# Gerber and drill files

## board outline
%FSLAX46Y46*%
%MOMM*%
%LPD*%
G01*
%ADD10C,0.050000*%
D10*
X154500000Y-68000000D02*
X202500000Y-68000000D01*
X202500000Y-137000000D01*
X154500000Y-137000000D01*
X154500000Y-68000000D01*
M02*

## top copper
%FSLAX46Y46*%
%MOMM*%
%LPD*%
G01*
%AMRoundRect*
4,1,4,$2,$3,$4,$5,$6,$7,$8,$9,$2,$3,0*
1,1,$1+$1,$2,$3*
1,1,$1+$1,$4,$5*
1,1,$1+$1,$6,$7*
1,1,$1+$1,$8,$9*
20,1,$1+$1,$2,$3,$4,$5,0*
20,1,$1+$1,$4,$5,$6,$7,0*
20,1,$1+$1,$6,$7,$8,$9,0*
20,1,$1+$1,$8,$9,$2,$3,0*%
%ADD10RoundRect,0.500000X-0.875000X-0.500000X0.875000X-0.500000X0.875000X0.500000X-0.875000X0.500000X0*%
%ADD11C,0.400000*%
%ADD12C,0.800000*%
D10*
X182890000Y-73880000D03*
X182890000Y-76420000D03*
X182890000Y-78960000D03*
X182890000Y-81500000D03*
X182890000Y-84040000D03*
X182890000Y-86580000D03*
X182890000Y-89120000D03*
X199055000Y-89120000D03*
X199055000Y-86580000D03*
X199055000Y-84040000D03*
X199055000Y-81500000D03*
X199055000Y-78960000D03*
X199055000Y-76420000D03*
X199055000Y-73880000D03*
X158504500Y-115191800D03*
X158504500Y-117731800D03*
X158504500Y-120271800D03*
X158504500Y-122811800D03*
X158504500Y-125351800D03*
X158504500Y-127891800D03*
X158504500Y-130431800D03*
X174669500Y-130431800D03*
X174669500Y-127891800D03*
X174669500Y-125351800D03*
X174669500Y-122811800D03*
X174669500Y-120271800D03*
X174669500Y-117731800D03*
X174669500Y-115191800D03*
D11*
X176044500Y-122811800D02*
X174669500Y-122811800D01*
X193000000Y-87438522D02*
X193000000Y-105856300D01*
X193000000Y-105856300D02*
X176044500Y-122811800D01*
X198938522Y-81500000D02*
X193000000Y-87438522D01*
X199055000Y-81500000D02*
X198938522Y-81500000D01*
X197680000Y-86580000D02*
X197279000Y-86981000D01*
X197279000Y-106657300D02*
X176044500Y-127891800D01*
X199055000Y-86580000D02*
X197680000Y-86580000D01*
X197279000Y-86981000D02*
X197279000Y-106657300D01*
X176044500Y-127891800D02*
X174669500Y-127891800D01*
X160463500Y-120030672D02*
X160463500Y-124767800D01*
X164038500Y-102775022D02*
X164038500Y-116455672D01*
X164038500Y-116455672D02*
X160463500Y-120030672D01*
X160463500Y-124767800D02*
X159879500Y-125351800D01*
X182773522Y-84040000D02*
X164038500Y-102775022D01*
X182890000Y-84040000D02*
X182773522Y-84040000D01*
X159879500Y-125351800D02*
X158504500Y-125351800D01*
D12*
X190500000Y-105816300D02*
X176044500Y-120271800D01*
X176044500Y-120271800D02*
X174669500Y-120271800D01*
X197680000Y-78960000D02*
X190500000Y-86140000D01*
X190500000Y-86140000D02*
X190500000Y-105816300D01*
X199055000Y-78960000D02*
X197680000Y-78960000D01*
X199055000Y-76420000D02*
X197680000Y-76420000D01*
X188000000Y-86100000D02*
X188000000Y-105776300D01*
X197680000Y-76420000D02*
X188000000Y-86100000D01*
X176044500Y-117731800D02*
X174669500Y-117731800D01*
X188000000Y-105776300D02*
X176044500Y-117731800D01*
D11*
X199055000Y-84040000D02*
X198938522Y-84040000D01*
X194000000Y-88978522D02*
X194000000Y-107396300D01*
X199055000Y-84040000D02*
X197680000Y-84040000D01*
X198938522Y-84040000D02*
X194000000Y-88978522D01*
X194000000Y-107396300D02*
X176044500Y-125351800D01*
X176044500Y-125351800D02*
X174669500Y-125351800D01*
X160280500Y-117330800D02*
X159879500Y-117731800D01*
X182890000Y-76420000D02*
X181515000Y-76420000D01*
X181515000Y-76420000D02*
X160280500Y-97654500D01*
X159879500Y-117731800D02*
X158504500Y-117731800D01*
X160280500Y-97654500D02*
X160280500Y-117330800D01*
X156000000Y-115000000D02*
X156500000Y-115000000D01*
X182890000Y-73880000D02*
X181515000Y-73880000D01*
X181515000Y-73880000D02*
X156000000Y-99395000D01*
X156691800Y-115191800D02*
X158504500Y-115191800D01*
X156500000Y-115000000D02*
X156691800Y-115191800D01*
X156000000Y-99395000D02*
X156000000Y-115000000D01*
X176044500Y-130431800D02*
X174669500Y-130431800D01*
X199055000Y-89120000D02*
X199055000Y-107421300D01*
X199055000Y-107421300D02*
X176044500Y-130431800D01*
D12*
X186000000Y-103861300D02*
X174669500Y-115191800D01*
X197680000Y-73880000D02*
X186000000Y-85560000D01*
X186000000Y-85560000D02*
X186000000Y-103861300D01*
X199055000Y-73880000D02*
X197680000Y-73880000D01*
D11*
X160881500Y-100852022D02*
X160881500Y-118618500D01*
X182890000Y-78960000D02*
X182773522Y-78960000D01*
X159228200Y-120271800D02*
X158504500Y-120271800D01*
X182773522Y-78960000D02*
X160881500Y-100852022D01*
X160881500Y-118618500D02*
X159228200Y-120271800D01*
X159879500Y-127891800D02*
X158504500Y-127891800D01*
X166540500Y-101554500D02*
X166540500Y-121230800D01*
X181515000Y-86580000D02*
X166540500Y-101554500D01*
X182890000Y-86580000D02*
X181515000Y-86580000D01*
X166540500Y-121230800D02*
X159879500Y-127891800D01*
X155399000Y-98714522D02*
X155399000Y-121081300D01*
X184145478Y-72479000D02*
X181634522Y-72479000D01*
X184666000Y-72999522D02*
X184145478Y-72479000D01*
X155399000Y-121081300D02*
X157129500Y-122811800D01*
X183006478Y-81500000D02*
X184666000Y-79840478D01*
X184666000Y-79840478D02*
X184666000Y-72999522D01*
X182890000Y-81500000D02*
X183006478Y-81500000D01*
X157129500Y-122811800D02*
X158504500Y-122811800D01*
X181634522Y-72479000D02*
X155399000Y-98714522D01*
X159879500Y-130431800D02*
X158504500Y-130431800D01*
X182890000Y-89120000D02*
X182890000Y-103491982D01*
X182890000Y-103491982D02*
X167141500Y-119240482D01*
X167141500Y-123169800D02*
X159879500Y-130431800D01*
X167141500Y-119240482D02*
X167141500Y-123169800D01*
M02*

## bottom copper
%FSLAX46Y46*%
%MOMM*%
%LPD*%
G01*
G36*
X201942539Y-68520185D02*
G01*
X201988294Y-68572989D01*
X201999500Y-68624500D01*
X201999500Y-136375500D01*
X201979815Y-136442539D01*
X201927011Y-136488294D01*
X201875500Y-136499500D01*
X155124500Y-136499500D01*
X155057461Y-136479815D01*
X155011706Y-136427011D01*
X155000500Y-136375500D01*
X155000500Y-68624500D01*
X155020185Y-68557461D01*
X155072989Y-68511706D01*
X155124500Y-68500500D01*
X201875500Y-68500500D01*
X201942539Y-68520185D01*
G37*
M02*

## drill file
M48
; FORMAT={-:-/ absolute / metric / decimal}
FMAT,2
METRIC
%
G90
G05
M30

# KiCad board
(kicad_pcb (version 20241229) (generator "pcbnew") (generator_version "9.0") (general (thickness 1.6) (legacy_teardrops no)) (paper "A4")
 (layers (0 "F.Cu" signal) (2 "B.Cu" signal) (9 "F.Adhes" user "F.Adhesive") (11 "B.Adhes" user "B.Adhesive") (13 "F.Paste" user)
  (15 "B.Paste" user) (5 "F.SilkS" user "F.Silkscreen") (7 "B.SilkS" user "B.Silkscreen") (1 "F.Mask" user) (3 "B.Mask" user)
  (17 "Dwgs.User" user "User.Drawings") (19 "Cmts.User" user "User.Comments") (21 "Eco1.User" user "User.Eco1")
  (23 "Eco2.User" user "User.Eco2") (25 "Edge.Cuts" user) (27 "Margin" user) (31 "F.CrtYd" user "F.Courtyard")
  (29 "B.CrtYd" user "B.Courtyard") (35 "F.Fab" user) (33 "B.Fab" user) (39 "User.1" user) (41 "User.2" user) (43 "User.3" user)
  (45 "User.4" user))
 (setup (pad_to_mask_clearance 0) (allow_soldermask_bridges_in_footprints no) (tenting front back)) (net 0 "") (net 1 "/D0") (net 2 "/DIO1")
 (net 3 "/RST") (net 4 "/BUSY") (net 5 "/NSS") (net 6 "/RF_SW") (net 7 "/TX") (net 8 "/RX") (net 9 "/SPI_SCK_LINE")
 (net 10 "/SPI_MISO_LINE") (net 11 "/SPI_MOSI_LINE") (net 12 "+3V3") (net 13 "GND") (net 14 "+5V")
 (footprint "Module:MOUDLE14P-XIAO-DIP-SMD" (layer "F.Cu") (at 191 81.5)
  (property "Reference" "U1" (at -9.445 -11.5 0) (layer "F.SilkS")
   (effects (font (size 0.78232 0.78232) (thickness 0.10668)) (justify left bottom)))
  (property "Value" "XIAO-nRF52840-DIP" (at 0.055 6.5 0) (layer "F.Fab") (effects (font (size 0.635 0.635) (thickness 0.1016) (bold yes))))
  (pad "1" smd roundrect (at -8.11 -7.62) (size 2.75 2) (layers "F.Cu" "F.Mask" "F.Paste") (roundrect_rratio 0.25) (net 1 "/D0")
   (solder_mask_margin 0.0508) (thermal_bridge_angle 45))
  (pad "2" smd roundrect (at -8.11 -5.08) (size 2.75 2) (layers "F.Cu" "F.Mask" "F.Paste") (roundrect_rratio 0.25) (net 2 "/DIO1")
   (solder_mask_margin 0.0508) (thermal_bridge_angle 45))
  (pad "3" smd roundrect (at -8.11 -2.54) (size 2.75 2) (layers "F.Cu" "F.Mask" "F.Paste") (roundrect_rratio 0.25) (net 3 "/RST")
   (solder_mask_margin 0.0508) (thermal_bridge_angle 45))
  (pad "4" smd roundrect (at -8.11 0) (size 2.75 2) (layers "F.Cu" "F.Mask" "F.Paste") (roundrect_rratio 0.25) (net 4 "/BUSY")
   (solder_mask_margin 0.0508) (thermal_bridge_angle 45))
  (pad "5" smd roundrect (at -8.11 2.54) (size 2.75 2) (layers "F.Cu" "F.Mask" "F.Paste") (roundrect_rratio 0.25) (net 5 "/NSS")
   (solder_mask_margin 0.0508) (thermal_bridge_angle 45))
  (pad "6" smd roundrect (at -8.11 5.08) (size 2.75 2) (layers "F.Cu" "F.Mask" "F.Paste") (roundrect_rratio 0.25) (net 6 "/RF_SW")
   (solder_mask_margin 0.0508) (thermal_bridge_angle 45))
  (pad "7" smd roundrect (at -8.11 7.62) (size 2.75 2) (layers "F.Cu" "F.Mask" "F.Paste") (roundrect_rratio 0.25) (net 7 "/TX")
   (solder_mask_margin 0.0508) (thermal_bridge_angle 45))
  (pad "8" smd roundrect (at 8.055 7.62) (size 2.75 2) (layers "F.Cu" "F.Mask" "F.Paste") (roundrect_rratio 0.25) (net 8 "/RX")
   (solder_mask_margin 0.0508) (thermal_bridge_angle 45))
  (pad "9" smd roundrect (at 8.055 5.08) (size 2.75 2) (layers "F.Cu" "F.Mask" "F.Paste") (roundrect_rratio 0.25) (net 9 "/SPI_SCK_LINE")
   (solder_mask_margin 0.0508) (thermal_bridge_angle 45))
  (pad "10" smd roundrect (at 8.055 2.54) (size 2.75 2) (layers "F.Cu" "F.Mask" "F.Paste") (roundrect_rratio 0.25) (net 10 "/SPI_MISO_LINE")
   (solder_mask_margin 0.0508) (thermal_bridge_angle 45))
  (pad "11" smd roundrect (at 8.055 0) (size 2.75 2) (layers "F.Cu" "F.Mask" "F.Paste") (roundrect_rratio 0.25) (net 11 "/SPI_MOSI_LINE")
   (solder_mask_margin 0.0508) (thermal_bridge_angle 45))
  (pad "12" smd roundrect (at 8.055 -2.54) (size 2.75 2) (layers "F.Cu" "F.Mask" "F.Paste") (roundrect_rratio 0.25) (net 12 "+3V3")
   (solder_mask_margin 0.0508) (thermal_bridge_angle 45))
  (pad "13" smd roundrect (at 8.055 -5.08) (size 2.75 2) (layers "F.Cu" "F.Mask" "F.Paste") (roundrect_rratio 0.25) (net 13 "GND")
   (solder_mask_margin 0.0508) (thermal_bridge_angle 45))
  (pad "14" smd roundrect (at 8.055 -7.62) (size 2.75 2) (layers "F.Cu" "F.Mask" "F.Paste") (roundrect_rratio 0.25) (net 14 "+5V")
   (solder_mask_margin 0.0508) (thermal_bridge_angle 45)))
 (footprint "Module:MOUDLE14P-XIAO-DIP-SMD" (layer "F.Cu") (at 166.6145 122.8118)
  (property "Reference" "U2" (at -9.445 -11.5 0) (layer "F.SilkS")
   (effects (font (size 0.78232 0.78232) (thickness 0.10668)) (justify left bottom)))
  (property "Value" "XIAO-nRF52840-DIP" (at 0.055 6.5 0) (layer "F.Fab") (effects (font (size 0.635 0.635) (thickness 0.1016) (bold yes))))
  (pad "1" smd roundrect (at -8.11 -7.62) (size 2.75 2) (layers "F.Cu" "F.Mask" "F.Paste") (roundrect_rratio 0.25) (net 1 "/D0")
   (solder_mask_margin 0.0508) (thermal_bridge_angle 45))
  (pad "2" smd roundrect (at -8.11 -5.08) (size 2.75 2) (layers "F.Cu" "F.Mask" "F.Paste") (roundrect_rratio 0.25) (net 2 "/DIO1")
   (solder_mask_margin 0.0508) (thermal_bridge_angle 45))
  (pad "3" smd roundrect (at -8.11 -2.54) (size 2.75 2) (layers "F.Cu" "F.Mask" "F.Paste") (roundrect_rratio 0.25) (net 3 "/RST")
   (solder_mask_margin 0.0508) (thermal_bridge_angle 45))
  (pad "4" smd roundrect (at -8.11 0) (size 2.75 2) (layers "F.Cu" "F.Mask" "F.Paste") (roundrect_rratio 0.25) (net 4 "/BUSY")
   (solder_mask_margin 0.0508) (thermal_bridge_angle 45))
  (pad "5" smd roundrect (at -8.11 2.54) (size 2.75 2) (layers "F.Cu" "F.Mask" "F.Paste") (roundrect_rratio 0.25) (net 5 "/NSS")
   (solder_mask_margin 0.0508) (thermal_bridge_angle 45))
  (pad "6" smd roundrect (at -8.11 5.08) (size 2.75 2) (layers "F.Cu" "F.Mask" "F.Paste") (roundrect_rratio 0.25) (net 6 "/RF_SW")
   (solder_mask_margin 0.0508) (thermal_bridge_angle 45))
  (pad "7" smd roundrect (at -8.11 7.62) (size 2.75 2) (layers "F.Cu" "F.Mask" "F.Paste") (roundrect_rratio 0.25) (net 7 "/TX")
   (solder_mask_margin 0.0508) (thermal_bridge_angle 45))
  (pad "8" smd roundrect (at 8.055 7.62) (size 2.75 2) (layers "F.Cu" "F.Mask" "F.Paste") (roundrect_rratio 0.25) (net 8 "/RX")
   (solder_mask_margin 0.0508) (thermal_bridge_angle 45))
  (pad "9" smd roundrect (at 8.055 5.08) (size 2.75 2) (layers "F.Cu" "F.Mask" "F.Paste") (roundrect_rratio 0.25) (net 9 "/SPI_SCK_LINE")
   (solder_mask_margin 0.0508) (thermal_bridge_angle 45))
  (pad "10" smd roundrect (at 8.055 2.54) (size 2.75 2) (layers "F.Cu" "F.Mask" "F.Paste") (roundrect_rratio 0.25) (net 10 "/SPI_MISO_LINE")
   (solder_mask_margin 0.0508) (thermal_bridge_angle 45))
  (pad "11" smd roundrect (at 8.055 0) (size 2.75 2) (layers "F.Cu" "F.Mask" "F.Paste") (roundrect_rratio 0.25) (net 11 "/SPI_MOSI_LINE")
   (solder_mask_margin 0.0508) (thermal_bridge_angle 45))
  (pad "12" smd roundrect (at 8.055 -2.54) (size 2.75 2) (layers "F.Cu" "F.Mask" "F.Paste") (roundrect_rratio 0.25) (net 12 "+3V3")
   (solder_mask_margin 0.0508) (thermal_bridge_angle 45))
  (pad "13" smd roundrect (at 8.055 -5.08) (size 2.75 2) (layers "F.Cu" "F.Mask" "F.Paste") (roundrect_rratio 0.25) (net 13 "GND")
   (solder_mask_margin 0.0508) (thermal_bridge_angle 45))
  (pad "14" smd roundrect (at 8.055 -7.62) (size 2.75 2) (layers "F.Cu" "F.Mask" "F.Paste") (roundrect_rratio 0.25) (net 14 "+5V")
   (solder_mask_margin 0.0508) (thermal_bridge_angle 45)))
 (gr_rect (start 154.5 68) (end 202.5 137) (stroke (width 0.05) (type default)) (fill no) (layer "Edge.Cuts"))
 (segment (start 176.0445 122.8118) (end 174.6695 122.8118) (width 0.4) (layer "F.Cu") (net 11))
 (segment (start 193 87.438522) (end 193 105.8563) (width 0.4) (layer "F.Cu") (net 11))
 (segment (start 193 105.8563) (end 176.0445 122.8118) (width 0.4) (layer "F.Cu") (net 11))
 (segment (start 198.938522 81.5) (end 193 87.438522) (width 0.4) (layer "F.Cu") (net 11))
 (segment (start 199.055 81.5) (end 198.938522 81.5) (width 0.4) (layer "F.Cu") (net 11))
 (segment (start 197.68 86.58) (end 197.279 86.981) (width 0.4) (layer "F.Cu") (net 9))
 (segment (start 197.279 106.6573) (end 176.0445 127.8918) (width 0.4) (layer "F.Cu") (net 9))
 (segment (start 199.055 86.58) (end 197.68 86.58) (width 0.4) (layer "F.Cu") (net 9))
 (segment (start 197.279 86.981) (end 197.279 106.6573) (width 0.4) (layer "F.Cu") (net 9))
 (segment (start 176.0445 127.8918) (end 174.6695 127.8918) (width 0.4) (layer "F.Cu") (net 9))
 (segment (start 160.4635 120.030672) (end 160.4635 124.7678) (width 0.4) (layer "F.Cu") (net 5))
 (segment (start 164.0385 102.775022) (end 164.0385 116.455672) (width 0.4) (layer "F.Cu") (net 5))
 (segment (start 164.0385 116.455672) (end 160.4635 120.030672) (width 0.4) (layer "F.Cu") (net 5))
 (segment (start 160.4635 124.7678) (end 159.8795 125.3518) (width 0.4) (layer "F.Cu") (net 5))
 (segment (start 182.773522 84.04) (end 164.0385 102.775022) (width 0.4) (layer "F.Cu") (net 5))
 (segment (start 182.89 84.04) (end 182.773522 84.04) (width 0.4) (layer "F.Cu") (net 5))
 (segment (start 159.8795 125.3518) (end 158.5045 125.3518) (width 0.4) (layer "F.Cu") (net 5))
 (segment (start 190.5 105.8163) (end 176.0445 120.2718) (width 0.8) (layer "F.Cu") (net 12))
 (segment (start 176.0445 120.2718) (end 174.6695 120.2718) (width 0.8) (layer "F.Cu") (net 12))
 (segment (start 197.68 78.96) (end 190.5 86.14) (width 0.8) (layer "F.Cu") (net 12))
 (segment (start 190.5 86.14) (end 190.5 105.8163) (width 0.8) (layer "F.Cu") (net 12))
 (segment (start 199.055 78.96) (end 197.68 78.96) (width 0.8) (layer "F.Cu") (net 12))
 (segment (start 199.055 76.42) (end 197.68 76.42) (width 0.8) (layer "F.Cu") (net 13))
 (segment (start 188 86.1) (end 188 105.7763) (width 0.8) (layer "F.Cu") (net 13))
 (segment (start 197.68 76.42) (end 188 86.1) (width 0.8) (layer "F.Cu") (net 13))
 (segment (start 176.0445 117.7318) (end 174.6695 117.7318) (width 0.8) (layer "F.Cu") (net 13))
 (segment (start 188 105.7763) (end 176.0445 117.7318) (width 0.8) (layer "F.Cu") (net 13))
 (segment (start 199.055 84.04) (end 198.938522 84.04) (width 0.4) (layer "F.Cu") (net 10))
 (segment (start 194 88.978522) (end 194 107.3963) (width 0.4) (layer "F.Cu") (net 10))
 (segment (start 199.055 84.04) (end 197.68 84.04) (width 0.4) (layer "F.Cu") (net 10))
 (segment (start 198.938522 84.04) (end 194 88.978522) (width 0.4) (layer "F.Cu") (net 10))
 (segment (start 194 107.3963) (end 176.0445 125.3518) (width 0.4) (layer "F.Cu") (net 10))
 (segment (start 176.0445 125.3518) (end 174.6695 125.3518) (width 0.4) (layer "F.Cu") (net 10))
 (segment (start 160.2805 117.3308) (end 159.8795 117.7318) (width 0.4) (layer "F.Cu") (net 2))
 (segment (start 182.89 76.42) (end 181.515 76.42) (width 0.4) (layer "F.Cu") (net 2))
 (segment (start 181.515 76.42) (end 160.2805 97.6545) (width 0.4) (layer "F.Cu") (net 2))
 (segment (start 159.8795 117.7318) (end 158.5045 117.7318) (width 0.4) (layer "F.Cu") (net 2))
 (segment (start 160.2805 97.6545) (end 160.2805 117.3308) (width 0.4) (layer "F.Cu") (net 2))
 (segment (start 156 115) (end 156.5 115) (width 0.4) (layer "F.Cu") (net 1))
 (segment (start 182.89 73.88) (end 181.515 73.88) (width 0.4) (layer "F.Cu") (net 1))
 (segment (start 181.515 73.88) (end 156 99.395) (width 0.4) (layer "F.Cu") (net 1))
 (segment (start 156.6918 115.1918) (end 158.5045 115.1918) (width 0.4) (layer "F.Cu") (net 1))
 (segment (start 156.5 115) (end 156.6918 115.1918) (width 0.4) (layer "F.Cu") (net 1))
 (segment (start 156 99.395) (end 156 115) (width 0.4) (layer "F.Cu") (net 1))
 (segment (start 176.0445 130.4318) (end 174.6695 130.4318) (width 0.4) (layer "F.Cu") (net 8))
 (segment (start 199.055 89.12) (end 199.055 107.4213) (width 0.4) (layer "F.Cu") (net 8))
 (segment (start 199.055 107.4213) (end 176.0445 130.4318) (width 0.4) (layer "F.Cu") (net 8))
 (segment (start 186 103.8613) (end 174.6695 115.1918) (width 0.8) (layer "F.Cu") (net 14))
 (segment (start 197.68 73.88) (end 186 85.56) (width 0.8) (layer "F.Cu") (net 14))
 (segment (start 186 85.56) (end 186 103.8613) (width 0.8) (layer "F.Cu") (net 14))
 (segment (start 199.055 73.88) (end 197.68 73.88) (width 0.8) (layer "F.Cu") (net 14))
 (segment (start 160.8815 100.852022) (end 160.8815 118.6185) (width 0.4) (layer "F.Cu") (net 3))
 (segment (start 182.89 78.96) (end 182.773522 78.96) (width 0.4) (layer "F.Cu") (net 3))
 (segment (start 159.2282 120.2718) (end 158.5045 120.2718) (width 0.4) (layer "F.Cu") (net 3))
 (segment (start 182.773522 78.96) (end 160.8815 100.852022) (width 0.4) (layer "F.Cu") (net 3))
 (segment (start 160.8815 118.6185) (end 159.2282 120.2718) (width 0.4) (layer "F.Cu") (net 3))
 (segment (start 159.8795 127.8918) (end 158.5045 127.8918) (width 0.4) (layer "F.Cu") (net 6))
 (segment (start 166.5405 101.5545) (end 166.5405 121.2308) (width 0.4) (layer "F.Cu") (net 6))
 (segment (start 181.515 86.58) (end 166.5405 101.5545) (width 0.4) (layer "F.Cu") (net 6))
 (segment (start 182.89 86.58) (end 181.515 86.58) (width 0.4) (layer "F.Cu") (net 6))
 (segment (start 166.5405 121.2308) (end 159.8795 127.8918) (width 0.4) (layer "F.Cu") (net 6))
 (segment (start 155.399 98.714522) (end 155.399 121.0813) (width 0.4) (layer "F.Cu") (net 4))
 (segment (start 184.145478 72.479) (end 181.634522 72.479) (width 0.4) (layer "F.Cu") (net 4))
 (segment (start 184.666 72.999522) (end 184.145478 72.479) (width 0.4) (layer "F.Cu") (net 4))
 (segment (start 155.399 121.0813) (end 157.1295 122.8118) (width 0.4) (layer "F.Cu") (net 4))
 (segment (start 183.006478 81.5) (end 184.666 79.840478) (width 0.4) (layer "F.Cu") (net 4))
 (segment (start 184.666 79.840478) (end 184.666 72.999522) (width 0.4) (layer "F.Cu") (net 4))
 (segment (start 182.89 81.5) (end 183.006478 81.5) (width 0.4) (layer "F.Cu") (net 4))
 (segment (start 157.1295 122.8118) (end 158.5045 122.8118) (width 0.4) (layer "F.Cu") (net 4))
 (segment (start 181.634522 72.479) (end 155.399 98.714522) (width 0.4) (layer "F.Cu") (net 4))
 (segment (start 159.8795 130.4318) (end 158.5045 130.4318) (width 0.4) (layer "F.Cu") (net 7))
 (segment (start 182.89 89.12) (end 182.89 103.491982) (width 0.4) (layer "F.Cu") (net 7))
 (segment (start 182.89 103.491982) (end 167.1415 119.240482) (width 0.4) (layer "F.Cu") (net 7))
 (segment (start 167.1415 123.1698) (end 159.8795 130.4318) (width 0.4) (layer "F.Cu") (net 7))
 (segment (start 167.1415 119.240482) (end 167.1415 123.1698) (width 0.4) (layer "F.Cu") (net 7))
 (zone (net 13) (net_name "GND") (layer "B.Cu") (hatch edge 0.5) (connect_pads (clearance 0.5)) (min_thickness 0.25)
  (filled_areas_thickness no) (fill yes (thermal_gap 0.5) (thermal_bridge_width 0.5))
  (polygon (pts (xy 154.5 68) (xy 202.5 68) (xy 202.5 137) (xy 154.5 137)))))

